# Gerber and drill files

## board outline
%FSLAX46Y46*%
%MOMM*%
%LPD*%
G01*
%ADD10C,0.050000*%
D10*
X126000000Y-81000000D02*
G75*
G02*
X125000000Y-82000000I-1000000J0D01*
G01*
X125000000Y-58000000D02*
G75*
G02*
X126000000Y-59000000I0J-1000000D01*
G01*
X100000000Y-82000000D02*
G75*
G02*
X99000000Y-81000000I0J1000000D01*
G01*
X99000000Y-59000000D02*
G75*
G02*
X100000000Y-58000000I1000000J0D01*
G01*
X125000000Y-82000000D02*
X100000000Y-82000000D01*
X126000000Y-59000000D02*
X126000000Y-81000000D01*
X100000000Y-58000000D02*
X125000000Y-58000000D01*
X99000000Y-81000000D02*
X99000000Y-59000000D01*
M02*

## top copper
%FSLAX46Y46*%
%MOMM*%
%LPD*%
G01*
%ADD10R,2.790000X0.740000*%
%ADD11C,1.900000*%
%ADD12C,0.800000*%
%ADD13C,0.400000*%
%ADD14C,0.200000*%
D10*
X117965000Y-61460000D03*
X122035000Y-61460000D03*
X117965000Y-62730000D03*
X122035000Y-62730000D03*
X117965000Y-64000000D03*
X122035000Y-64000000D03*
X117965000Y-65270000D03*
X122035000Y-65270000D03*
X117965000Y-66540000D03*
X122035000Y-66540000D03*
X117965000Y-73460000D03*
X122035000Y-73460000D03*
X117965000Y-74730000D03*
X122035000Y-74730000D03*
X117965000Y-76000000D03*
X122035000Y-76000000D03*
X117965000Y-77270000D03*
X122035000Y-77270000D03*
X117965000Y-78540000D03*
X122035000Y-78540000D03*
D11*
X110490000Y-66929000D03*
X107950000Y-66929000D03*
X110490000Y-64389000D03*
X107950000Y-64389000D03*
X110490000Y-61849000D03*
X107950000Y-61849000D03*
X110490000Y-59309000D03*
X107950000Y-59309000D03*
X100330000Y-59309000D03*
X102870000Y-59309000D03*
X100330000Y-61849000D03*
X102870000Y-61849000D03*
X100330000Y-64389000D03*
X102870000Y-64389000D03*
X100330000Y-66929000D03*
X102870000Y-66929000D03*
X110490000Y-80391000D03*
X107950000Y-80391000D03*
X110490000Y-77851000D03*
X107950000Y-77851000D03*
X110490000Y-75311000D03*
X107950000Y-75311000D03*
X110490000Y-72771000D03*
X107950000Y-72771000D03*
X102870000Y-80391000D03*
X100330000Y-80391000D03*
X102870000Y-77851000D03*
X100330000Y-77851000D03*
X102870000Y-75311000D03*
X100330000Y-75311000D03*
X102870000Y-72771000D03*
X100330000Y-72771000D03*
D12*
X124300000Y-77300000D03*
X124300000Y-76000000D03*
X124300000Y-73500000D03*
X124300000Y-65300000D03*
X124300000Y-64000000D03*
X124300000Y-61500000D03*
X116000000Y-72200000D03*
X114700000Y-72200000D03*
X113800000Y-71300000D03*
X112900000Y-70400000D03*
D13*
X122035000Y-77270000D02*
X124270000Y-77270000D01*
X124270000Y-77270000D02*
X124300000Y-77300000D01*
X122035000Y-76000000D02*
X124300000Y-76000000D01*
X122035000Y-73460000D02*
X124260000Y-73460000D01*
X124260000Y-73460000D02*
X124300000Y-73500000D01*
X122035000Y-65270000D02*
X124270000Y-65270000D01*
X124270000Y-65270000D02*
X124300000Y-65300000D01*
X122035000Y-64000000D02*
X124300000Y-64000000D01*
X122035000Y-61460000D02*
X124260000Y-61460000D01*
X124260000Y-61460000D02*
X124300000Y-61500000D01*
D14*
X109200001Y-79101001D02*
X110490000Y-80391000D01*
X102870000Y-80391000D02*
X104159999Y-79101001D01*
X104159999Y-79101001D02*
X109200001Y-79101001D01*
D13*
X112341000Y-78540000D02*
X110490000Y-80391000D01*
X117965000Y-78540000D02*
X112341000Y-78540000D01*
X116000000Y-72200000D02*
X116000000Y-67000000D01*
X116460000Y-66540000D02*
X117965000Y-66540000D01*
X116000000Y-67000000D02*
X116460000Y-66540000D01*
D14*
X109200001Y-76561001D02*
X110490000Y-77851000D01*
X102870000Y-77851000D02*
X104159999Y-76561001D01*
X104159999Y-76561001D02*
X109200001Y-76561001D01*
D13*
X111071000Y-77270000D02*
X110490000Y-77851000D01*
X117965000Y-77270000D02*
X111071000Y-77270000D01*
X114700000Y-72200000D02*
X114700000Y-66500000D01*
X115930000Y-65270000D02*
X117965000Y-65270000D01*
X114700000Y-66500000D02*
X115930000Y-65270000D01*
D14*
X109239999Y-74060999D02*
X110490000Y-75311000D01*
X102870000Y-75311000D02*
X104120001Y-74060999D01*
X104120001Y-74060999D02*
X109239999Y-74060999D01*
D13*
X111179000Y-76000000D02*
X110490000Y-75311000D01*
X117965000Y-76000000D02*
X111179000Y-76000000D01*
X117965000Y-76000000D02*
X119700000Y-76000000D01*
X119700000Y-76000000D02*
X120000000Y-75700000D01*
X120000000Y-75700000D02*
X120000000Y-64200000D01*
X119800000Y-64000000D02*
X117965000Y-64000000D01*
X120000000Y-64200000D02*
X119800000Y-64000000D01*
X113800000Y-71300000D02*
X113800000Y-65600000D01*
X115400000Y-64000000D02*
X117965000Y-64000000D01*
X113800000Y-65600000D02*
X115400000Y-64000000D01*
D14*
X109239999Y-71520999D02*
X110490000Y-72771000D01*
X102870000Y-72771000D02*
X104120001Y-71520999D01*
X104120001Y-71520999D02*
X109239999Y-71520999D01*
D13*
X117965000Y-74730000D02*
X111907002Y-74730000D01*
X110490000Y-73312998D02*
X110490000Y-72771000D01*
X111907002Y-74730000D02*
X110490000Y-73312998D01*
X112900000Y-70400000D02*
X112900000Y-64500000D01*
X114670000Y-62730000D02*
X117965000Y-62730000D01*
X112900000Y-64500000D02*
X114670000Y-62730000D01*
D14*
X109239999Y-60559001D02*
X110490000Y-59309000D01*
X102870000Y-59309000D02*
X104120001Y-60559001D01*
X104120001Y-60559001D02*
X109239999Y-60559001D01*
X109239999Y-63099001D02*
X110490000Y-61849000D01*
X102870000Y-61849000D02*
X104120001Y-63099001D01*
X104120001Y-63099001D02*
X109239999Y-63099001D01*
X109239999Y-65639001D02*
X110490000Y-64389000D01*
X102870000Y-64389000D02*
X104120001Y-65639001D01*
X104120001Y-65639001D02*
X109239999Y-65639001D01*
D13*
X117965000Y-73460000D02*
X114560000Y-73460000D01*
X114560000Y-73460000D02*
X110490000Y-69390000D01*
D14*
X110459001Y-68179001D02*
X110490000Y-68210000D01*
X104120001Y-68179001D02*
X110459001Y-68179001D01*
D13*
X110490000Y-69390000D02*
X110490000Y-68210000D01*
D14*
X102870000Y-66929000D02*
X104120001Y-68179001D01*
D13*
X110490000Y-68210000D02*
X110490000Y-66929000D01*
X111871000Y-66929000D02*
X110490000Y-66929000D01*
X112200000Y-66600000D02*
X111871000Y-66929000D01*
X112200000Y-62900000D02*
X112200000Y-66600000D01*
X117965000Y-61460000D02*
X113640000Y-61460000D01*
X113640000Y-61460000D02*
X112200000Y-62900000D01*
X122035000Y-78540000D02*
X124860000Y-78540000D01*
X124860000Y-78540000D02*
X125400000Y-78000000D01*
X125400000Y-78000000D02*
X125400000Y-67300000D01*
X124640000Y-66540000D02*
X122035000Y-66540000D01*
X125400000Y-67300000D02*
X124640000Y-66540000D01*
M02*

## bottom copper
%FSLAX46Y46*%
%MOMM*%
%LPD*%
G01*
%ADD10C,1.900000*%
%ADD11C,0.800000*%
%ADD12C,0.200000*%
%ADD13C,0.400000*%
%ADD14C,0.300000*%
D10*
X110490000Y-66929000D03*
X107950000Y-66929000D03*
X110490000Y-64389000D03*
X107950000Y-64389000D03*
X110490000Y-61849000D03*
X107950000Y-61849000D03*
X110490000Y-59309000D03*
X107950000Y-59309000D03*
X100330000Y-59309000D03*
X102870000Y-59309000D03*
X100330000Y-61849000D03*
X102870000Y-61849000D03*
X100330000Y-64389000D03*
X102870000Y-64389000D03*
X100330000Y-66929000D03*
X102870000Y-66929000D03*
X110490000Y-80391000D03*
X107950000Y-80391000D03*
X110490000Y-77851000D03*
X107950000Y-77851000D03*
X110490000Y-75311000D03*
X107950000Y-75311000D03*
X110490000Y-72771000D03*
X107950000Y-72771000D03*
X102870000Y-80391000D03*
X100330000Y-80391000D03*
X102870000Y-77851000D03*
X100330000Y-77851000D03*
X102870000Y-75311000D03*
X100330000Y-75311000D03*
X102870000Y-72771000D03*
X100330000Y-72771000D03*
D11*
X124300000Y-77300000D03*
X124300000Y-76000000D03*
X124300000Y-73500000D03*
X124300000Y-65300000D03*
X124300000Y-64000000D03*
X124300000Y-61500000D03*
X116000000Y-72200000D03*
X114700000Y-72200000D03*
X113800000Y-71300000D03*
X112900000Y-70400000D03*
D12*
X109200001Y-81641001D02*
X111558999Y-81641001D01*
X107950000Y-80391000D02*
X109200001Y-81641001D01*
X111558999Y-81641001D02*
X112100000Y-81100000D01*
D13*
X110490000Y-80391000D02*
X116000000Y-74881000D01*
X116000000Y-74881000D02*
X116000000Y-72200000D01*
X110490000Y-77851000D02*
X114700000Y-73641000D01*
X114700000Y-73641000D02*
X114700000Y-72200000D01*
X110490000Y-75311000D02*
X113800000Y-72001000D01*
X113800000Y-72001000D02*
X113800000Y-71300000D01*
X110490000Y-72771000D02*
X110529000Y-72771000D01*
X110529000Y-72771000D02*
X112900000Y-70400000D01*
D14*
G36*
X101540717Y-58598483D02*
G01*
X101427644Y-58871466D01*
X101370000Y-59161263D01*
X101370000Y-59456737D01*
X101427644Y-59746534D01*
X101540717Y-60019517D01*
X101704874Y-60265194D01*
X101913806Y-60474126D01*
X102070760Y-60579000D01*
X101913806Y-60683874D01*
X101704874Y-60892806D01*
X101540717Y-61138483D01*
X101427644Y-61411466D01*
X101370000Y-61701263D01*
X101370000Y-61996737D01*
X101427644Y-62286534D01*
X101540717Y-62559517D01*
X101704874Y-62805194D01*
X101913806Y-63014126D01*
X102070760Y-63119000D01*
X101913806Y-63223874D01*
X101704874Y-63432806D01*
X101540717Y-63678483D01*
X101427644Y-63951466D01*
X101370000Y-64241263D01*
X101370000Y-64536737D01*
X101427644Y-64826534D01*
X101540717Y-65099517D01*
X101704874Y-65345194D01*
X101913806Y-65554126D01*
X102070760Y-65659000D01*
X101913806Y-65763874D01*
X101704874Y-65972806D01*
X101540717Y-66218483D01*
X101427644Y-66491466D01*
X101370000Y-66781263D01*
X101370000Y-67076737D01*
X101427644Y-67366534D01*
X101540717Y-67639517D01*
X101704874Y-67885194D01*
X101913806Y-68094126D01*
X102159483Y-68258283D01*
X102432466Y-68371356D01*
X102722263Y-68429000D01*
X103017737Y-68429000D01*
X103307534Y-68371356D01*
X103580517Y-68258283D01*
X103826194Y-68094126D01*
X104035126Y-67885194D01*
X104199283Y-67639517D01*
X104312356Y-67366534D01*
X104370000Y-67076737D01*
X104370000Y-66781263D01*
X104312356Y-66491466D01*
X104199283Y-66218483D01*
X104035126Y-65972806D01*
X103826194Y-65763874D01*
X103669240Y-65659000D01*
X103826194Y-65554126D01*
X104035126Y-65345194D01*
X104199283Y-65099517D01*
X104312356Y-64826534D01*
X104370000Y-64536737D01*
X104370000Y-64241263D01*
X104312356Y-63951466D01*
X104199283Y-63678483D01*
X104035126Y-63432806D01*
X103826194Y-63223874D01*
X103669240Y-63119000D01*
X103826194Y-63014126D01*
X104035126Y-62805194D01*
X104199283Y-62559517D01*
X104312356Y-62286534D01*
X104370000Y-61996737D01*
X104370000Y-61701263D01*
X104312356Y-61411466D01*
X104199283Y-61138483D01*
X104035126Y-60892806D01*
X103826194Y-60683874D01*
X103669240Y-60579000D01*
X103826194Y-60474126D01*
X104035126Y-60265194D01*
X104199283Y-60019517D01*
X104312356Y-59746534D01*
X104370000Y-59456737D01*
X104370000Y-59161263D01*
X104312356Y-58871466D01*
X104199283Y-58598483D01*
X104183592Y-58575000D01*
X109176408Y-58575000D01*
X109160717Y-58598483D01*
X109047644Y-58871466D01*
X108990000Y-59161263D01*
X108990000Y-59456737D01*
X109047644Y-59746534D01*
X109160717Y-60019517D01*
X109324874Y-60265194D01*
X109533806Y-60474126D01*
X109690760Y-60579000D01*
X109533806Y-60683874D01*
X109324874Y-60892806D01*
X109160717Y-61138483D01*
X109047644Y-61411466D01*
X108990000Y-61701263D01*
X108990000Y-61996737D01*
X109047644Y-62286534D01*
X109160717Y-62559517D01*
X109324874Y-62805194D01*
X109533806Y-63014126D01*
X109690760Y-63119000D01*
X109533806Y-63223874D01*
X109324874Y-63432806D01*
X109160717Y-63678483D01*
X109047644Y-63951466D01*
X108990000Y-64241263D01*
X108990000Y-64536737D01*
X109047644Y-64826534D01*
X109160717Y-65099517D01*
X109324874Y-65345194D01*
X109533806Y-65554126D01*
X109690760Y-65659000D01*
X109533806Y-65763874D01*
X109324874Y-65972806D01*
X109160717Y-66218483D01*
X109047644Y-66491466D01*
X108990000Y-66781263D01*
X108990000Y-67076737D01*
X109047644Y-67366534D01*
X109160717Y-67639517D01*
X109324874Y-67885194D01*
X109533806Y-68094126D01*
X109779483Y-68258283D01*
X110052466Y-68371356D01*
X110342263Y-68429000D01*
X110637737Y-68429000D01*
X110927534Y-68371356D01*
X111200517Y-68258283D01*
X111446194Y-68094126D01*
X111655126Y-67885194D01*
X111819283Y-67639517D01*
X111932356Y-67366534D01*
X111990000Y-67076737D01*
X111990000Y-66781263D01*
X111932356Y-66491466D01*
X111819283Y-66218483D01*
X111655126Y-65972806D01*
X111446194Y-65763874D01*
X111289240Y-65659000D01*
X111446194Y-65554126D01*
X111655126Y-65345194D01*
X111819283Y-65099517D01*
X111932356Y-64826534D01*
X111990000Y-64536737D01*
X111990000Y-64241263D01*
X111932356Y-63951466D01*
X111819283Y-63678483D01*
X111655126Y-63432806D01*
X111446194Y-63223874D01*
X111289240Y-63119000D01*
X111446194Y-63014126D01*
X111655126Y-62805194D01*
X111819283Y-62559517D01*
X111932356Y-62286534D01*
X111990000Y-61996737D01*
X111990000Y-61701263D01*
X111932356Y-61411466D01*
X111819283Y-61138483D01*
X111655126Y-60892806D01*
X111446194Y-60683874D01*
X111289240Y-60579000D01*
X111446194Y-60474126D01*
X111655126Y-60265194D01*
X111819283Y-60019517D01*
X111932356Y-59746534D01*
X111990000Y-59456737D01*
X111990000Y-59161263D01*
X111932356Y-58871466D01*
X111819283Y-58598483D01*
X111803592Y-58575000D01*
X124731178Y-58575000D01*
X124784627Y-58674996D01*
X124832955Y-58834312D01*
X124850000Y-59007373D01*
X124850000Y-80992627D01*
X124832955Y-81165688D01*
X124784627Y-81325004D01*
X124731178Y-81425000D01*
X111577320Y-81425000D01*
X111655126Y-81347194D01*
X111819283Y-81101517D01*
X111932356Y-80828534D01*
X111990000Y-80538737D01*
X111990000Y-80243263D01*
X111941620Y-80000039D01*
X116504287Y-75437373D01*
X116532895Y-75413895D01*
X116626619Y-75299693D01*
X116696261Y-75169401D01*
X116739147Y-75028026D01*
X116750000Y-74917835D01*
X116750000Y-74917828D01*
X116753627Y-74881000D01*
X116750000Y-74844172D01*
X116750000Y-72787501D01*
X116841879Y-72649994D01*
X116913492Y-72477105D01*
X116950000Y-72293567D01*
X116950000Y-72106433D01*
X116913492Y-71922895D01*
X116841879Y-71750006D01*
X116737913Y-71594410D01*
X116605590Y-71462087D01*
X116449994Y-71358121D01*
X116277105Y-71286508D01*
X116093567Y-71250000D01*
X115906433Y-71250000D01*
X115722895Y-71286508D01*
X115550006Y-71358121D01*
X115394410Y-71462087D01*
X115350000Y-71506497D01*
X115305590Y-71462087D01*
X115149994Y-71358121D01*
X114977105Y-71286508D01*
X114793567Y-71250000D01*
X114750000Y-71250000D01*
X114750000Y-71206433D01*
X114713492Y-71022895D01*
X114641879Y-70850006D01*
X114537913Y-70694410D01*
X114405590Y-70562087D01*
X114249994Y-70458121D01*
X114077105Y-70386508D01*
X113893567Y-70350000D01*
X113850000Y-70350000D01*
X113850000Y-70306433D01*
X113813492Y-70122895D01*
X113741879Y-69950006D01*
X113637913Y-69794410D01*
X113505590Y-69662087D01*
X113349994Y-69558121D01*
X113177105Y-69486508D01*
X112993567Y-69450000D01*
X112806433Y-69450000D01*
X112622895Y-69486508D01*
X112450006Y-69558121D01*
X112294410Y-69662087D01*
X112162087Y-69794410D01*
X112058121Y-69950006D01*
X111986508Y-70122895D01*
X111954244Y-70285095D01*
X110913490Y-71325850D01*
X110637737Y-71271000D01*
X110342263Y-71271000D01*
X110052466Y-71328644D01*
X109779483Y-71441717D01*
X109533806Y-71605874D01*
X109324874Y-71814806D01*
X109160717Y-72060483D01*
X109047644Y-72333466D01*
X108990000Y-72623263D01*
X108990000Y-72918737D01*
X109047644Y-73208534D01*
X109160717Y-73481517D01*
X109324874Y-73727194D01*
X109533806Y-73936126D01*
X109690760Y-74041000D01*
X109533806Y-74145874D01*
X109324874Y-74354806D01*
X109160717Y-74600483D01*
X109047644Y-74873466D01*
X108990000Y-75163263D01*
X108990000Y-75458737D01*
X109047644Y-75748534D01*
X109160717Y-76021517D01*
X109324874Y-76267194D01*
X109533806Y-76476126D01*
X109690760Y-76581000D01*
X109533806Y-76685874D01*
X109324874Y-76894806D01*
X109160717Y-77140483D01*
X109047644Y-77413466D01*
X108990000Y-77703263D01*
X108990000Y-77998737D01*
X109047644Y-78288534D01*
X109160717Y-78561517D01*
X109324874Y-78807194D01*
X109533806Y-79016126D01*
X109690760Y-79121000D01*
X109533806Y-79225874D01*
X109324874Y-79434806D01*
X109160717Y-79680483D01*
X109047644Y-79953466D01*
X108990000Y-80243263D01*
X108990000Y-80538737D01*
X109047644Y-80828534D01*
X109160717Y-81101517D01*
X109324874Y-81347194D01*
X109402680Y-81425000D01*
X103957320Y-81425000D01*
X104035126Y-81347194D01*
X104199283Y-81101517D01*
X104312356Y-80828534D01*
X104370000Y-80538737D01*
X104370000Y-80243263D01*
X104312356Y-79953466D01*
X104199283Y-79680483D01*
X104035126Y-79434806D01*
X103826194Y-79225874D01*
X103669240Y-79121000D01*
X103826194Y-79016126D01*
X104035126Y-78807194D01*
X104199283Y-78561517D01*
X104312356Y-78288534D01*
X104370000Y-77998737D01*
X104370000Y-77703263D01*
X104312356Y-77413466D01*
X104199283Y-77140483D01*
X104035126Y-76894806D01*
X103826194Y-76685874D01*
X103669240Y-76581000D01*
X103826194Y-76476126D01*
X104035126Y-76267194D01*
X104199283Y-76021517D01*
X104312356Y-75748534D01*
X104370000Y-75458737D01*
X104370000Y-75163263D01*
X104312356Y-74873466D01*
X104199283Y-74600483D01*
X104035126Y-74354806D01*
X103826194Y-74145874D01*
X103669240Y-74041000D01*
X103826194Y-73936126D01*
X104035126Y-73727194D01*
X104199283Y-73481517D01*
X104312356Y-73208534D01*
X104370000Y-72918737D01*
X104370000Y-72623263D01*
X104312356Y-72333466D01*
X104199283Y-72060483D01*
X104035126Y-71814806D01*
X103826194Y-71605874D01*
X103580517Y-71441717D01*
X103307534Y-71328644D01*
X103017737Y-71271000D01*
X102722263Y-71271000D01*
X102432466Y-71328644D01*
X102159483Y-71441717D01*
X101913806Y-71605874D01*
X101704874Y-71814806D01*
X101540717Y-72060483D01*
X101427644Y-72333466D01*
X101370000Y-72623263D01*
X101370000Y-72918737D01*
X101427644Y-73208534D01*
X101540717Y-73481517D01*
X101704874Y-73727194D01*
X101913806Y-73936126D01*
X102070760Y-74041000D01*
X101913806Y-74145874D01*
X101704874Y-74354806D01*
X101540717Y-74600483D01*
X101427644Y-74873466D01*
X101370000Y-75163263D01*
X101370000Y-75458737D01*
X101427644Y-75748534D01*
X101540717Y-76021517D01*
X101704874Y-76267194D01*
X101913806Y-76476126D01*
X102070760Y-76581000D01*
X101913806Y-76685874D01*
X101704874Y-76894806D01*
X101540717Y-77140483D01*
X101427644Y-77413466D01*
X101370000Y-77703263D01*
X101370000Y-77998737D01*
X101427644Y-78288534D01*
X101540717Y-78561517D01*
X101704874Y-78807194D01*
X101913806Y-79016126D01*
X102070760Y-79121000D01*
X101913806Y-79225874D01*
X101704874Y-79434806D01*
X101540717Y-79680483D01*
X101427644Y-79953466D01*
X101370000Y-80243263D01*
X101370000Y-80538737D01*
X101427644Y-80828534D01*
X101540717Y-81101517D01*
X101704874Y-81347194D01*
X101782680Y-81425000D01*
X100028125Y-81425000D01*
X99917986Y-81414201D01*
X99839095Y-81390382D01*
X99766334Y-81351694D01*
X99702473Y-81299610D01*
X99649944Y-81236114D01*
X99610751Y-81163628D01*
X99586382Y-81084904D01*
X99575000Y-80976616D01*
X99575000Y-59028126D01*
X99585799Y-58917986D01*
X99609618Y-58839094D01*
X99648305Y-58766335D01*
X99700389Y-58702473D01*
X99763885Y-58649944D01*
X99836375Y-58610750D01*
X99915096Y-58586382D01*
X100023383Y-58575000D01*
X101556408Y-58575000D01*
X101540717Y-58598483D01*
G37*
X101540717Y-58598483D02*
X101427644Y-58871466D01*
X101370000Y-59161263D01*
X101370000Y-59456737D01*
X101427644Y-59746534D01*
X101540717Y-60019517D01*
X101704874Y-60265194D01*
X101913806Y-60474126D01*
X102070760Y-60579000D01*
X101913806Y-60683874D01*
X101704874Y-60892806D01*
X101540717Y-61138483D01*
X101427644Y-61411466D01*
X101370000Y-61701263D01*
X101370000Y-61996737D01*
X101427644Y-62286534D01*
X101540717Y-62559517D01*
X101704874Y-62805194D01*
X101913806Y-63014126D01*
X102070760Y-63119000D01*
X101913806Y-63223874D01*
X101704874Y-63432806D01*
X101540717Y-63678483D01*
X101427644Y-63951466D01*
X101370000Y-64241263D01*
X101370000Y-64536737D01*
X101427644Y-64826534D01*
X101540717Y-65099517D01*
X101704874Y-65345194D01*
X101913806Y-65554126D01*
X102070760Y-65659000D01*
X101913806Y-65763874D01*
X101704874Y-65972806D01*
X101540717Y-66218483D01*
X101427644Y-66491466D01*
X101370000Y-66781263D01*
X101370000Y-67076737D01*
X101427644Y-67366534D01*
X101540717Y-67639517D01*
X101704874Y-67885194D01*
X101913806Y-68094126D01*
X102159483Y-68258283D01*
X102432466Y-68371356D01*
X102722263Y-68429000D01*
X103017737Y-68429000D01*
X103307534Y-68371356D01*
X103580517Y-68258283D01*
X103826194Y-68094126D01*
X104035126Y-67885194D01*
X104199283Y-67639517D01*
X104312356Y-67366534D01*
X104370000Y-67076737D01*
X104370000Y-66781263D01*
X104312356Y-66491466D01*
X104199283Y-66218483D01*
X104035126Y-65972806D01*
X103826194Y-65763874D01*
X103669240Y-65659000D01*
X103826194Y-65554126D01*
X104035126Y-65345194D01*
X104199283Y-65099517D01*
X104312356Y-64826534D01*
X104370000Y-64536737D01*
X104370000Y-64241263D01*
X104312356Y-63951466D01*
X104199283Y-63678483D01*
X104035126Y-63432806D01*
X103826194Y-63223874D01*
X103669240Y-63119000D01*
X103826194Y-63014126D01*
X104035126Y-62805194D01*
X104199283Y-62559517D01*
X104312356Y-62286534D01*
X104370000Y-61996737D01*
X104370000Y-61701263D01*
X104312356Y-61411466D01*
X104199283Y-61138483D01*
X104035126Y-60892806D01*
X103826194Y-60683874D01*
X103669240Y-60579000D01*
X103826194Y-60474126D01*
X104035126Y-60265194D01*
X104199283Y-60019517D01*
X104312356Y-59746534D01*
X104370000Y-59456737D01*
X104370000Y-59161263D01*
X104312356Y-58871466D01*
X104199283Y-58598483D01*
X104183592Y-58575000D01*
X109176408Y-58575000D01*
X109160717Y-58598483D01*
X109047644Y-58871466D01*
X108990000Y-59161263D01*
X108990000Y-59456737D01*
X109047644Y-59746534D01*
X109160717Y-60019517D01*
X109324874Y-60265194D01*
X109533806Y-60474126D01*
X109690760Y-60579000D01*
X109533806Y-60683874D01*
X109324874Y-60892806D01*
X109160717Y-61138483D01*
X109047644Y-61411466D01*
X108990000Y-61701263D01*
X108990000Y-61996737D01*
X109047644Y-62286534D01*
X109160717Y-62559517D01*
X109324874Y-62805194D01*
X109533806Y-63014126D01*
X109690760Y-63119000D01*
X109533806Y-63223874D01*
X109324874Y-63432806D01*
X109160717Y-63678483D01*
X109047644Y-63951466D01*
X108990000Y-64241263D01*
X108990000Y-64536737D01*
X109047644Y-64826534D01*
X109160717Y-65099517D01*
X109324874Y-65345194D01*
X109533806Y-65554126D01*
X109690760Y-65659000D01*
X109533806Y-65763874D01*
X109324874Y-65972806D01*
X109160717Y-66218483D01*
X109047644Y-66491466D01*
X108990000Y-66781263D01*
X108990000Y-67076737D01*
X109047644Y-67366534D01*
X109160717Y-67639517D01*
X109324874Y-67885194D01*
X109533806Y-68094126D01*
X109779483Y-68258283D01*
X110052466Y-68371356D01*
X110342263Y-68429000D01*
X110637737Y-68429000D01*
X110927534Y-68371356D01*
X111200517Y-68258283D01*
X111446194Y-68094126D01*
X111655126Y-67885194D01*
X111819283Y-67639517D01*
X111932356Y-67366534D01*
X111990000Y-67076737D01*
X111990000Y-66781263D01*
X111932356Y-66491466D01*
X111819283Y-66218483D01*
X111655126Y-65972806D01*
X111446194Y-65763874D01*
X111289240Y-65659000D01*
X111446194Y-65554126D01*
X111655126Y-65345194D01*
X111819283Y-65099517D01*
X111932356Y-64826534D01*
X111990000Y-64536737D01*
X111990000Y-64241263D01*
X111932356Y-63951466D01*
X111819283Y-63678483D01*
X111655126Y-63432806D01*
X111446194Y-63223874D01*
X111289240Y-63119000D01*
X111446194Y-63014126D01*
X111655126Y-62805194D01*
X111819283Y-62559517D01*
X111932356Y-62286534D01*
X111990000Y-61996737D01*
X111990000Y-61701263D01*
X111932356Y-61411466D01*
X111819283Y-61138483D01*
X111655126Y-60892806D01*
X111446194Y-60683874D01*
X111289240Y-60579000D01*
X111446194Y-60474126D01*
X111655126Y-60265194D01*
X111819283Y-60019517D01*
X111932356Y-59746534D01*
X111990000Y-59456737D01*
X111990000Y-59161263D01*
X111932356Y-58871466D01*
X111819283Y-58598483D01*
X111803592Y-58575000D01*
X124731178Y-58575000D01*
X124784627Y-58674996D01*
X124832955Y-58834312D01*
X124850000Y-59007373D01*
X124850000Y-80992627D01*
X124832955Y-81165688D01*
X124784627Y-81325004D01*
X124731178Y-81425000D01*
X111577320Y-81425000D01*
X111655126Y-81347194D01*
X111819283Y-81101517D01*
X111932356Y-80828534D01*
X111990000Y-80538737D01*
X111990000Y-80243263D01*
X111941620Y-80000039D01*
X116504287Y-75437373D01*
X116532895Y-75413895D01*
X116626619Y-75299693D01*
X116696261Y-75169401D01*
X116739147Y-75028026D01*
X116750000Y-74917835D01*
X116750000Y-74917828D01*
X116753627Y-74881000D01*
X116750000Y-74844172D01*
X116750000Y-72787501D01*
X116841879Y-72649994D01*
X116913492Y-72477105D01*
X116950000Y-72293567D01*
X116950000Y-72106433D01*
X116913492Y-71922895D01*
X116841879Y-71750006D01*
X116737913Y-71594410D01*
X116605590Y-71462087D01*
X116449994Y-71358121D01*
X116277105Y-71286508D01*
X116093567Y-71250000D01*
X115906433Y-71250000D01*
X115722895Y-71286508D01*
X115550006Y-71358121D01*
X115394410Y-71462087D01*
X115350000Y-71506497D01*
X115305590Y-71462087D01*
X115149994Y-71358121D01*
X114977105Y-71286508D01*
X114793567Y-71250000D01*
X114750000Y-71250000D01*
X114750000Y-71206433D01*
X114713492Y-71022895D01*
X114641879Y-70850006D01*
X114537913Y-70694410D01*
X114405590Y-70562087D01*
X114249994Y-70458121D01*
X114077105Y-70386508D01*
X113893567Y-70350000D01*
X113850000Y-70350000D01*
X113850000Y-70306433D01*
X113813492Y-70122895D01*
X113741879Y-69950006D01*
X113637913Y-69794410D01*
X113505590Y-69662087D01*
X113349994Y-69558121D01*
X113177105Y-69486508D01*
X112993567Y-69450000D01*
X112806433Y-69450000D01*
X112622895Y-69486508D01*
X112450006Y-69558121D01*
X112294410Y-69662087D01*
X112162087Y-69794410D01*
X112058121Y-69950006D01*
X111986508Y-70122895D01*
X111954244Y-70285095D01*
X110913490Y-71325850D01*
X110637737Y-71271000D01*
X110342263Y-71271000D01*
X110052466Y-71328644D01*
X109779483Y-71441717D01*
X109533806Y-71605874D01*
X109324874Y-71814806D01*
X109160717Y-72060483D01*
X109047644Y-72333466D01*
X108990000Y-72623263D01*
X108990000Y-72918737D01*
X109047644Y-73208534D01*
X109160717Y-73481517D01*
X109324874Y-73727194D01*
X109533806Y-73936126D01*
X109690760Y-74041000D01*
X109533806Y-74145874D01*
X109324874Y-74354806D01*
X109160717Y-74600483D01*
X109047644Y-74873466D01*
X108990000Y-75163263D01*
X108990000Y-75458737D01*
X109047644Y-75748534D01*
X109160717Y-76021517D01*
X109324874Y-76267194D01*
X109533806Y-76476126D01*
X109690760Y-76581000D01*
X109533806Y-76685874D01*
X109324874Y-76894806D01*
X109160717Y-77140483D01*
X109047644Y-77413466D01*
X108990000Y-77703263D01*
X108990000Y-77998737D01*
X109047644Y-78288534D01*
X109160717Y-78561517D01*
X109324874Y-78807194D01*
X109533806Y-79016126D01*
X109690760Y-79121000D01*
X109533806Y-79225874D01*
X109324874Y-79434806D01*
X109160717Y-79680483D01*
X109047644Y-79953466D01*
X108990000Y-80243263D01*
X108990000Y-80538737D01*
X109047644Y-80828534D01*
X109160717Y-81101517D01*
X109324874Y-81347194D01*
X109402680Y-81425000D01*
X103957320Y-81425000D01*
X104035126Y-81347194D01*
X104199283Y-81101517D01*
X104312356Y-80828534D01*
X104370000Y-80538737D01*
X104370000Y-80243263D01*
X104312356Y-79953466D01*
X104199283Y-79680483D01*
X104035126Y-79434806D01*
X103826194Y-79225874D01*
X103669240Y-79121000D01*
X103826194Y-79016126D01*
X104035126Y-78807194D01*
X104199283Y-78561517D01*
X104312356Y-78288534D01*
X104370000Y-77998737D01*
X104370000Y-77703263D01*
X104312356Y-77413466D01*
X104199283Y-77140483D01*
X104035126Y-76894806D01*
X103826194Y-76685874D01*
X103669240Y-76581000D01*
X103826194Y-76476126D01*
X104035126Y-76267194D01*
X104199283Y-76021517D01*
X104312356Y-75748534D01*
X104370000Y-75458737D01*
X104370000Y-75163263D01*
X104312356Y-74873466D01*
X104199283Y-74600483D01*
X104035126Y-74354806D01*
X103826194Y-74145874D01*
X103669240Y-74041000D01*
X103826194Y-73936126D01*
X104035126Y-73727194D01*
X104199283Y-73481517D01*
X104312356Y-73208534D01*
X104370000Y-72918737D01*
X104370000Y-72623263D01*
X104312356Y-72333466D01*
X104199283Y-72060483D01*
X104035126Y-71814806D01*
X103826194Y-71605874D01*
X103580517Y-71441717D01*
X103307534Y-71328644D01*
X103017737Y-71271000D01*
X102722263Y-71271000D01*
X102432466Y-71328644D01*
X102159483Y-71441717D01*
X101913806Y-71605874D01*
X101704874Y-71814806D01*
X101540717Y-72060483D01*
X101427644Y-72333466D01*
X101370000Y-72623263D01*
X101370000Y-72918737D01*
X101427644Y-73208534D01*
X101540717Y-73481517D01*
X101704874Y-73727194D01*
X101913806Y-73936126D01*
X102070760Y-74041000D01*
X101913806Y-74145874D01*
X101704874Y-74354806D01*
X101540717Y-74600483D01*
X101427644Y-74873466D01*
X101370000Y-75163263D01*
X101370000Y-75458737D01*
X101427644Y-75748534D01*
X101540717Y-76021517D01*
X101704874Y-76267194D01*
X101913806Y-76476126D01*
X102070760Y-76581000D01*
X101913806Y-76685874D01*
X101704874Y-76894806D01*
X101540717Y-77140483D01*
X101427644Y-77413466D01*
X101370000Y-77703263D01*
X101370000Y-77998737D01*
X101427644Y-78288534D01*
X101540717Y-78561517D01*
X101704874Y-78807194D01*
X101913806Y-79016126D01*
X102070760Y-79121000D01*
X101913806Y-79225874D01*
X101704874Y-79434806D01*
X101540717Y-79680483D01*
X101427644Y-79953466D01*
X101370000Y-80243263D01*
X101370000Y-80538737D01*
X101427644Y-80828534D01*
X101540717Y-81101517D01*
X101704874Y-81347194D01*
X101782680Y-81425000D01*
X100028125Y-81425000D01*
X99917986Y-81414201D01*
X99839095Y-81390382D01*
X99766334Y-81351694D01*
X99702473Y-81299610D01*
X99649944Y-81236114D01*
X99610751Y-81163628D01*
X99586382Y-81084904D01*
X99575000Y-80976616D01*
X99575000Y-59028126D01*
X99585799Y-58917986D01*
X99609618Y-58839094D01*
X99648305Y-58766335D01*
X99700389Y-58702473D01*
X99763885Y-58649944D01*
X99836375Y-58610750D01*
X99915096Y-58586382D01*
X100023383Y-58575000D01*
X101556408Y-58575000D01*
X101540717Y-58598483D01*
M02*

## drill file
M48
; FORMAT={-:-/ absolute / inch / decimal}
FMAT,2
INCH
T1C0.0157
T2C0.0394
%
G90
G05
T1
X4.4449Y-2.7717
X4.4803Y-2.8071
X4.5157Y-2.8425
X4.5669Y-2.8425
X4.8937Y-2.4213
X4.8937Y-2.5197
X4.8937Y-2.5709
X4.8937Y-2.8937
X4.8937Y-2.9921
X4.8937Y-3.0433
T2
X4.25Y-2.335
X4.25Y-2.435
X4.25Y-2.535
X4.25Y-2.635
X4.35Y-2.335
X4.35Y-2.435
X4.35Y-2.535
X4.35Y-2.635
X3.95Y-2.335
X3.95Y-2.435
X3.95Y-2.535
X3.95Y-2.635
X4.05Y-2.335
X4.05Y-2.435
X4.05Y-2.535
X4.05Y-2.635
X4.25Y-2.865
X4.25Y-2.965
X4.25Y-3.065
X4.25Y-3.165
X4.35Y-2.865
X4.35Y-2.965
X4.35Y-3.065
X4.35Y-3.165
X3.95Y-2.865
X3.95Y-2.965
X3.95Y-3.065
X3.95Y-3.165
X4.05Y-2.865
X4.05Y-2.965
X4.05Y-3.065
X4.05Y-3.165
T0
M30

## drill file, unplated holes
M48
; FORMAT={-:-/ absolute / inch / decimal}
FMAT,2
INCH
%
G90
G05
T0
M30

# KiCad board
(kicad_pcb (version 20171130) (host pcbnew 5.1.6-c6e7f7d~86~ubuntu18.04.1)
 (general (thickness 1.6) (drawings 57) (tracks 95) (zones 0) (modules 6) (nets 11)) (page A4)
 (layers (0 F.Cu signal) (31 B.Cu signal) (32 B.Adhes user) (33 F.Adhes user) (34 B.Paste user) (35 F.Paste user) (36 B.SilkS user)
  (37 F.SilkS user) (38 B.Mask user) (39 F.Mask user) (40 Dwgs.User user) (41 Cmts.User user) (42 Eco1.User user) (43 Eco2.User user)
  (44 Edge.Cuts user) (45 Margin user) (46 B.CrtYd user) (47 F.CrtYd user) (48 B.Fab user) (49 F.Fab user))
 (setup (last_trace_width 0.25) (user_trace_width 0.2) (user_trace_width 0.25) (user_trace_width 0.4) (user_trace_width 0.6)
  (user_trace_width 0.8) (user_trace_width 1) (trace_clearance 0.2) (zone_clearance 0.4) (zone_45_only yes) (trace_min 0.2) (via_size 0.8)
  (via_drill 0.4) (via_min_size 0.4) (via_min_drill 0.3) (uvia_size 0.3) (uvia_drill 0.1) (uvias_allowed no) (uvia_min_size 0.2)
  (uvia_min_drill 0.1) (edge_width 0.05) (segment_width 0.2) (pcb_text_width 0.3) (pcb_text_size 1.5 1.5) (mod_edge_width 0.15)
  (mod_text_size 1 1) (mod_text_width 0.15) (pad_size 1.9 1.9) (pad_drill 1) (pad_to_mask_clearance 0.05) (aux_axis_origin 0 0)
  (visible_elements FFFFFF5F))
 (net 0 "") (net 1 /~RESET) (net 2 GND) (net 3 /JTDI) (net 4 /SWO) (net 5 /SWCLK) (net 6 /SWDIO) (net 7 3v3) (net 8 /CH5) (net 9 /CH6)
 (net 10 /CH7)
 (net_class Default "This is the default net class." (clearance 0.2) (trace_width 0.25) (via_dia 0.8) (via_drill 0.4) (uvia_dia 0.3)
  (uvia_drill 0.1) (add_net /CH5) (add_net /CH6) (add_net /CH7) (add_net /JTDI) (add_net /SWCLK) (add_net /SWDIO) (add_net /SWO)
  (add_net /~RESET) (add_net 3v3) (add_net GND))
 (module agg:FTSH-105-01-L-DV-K (layer F.Cu) (at 120 64 90)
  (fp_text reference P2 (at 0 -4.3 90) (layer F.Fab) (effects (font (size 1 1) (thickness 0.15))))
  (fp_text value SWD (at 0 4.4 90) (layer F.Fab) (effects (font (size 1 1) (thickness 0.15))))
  (pad 10 smd rect (at 2.54 -2.035 90) (size 0.74 2.79) (layers F.Cu F.Paste F.Mask) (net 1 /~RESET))
  (pad 9 smd rect (at 2.54 2.035 90) (size 0.74 2.79) (layers F.Cu F.Paste F.Mask) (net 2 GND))
  (pad 8 smd rect (at 1.27 -2.035 90) (size 0.74 2.79) (layers F.Cu F.Paste F.Mask) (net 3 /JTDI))
  (pad 7 smd rect (at 1.27 2.035 90) (size 0.74 2.79) (layers F.Cu F.Paste F.Mask))
  (pad 6 smd rect (at 0 -2.035 90) (size 0.74 2.79) (layers F.Cu F.Paste F.Mask) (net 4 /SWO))
  (pad 5 smd rect (at 0 2.035 90) (size 0.74 2.79) (layers F.Cu F.Paste F.Mask) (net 2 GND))
  (pad 4 smd rect (at -1.27 -2.035 90) (size 0.74 2.79) (layers F.Cu F.Paste F.Mask) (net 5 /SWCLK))
  (pad 3 smd rect (at -1.27 2.035 90) (size 0.74 2.79) (layers F.Cu F.Paste F.Mask) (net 2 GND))
  (pad 2 smd rect (at -2.54 -2.035 90) (size 0.74 2.79) (layers F.Cu F.Paste F.Mask) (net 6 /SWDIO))
  (pad 1 smd rect (at -2.54 2.035 90) (size 0.74 2.79) (layers F.Cu F.Paste F.Mask) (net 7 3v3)))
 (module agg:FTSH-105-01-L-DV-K (layer F.Cu) (at 120 76 90)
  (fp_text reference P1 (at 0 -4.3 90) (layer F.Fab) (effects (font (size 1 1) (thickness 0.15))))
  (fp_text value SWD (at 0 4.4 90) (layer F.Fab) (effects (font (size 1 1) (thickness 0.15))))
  (pad 10 smd rect (at 2.54 -2.035 90) (size 0.74 2.79) (layers F.Cu F.Paste F.Mask) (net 1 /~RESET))
  (pad 9 smd rect (at 2.54 2.035 90) (size 0.74 2.79) (layers F.Cu F.Paste F.Mask) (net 2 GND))
  (pad 8 smd rect (at 1.27 -2.035 90) (size 0.74 2.79) (layers F.Cu F.Paste F.Mask) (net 3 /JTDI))
  (pad 7 smd rect (at 1.27 2.035 90) (size 0.74 2.79) (layers F.Cu F.Paste F.Mask))
  (pad 6 smd rect (at 0 -2.035 90) (size 0.74 2.79) (layers F.Cu F.Paste F.Mask) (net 4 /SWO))
  (pad 5 smd rect (at 0 2.035 90) (size 0.74 2.79) (layers F.Cu F.Paste F.Mask) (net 2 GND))
  (pad 4 smd rect (at -1.27 -2.035 90) (size 0.74 2.79) (layers F.Cu F.Paste F.Mask) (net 5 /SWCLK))
  (pad 3 smd rect (at -1.27 2.035 90) (size 0.74 2.79) (layers F.Cu F.Paste F.Mask) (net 2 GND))
  (pad 2 smd rect (at -2.54 -2.035 90) (size 0.74 2.79) (layers F.Cu F.Paste F.Mask) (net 6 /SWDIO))
  (pad 1 smd rect (at -2.54 2.035 90) (size 0.74 2.79) (layers F.Cu F.Paste F.Mask) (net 7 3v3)))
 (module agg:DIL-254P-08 (layer F.Cu) (at 109.22 63.119 270)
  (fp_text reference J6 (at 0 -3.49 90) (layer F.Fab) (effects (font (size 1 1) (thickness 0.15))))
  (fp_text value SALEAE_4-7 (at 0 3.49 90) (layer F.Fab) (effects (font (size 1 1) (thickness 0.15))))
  (pad 8 thru_hole circle (at 3.81 -1.27 270) (size 1.9 1.9) (drill 1) (layers *.Cu *.Mask F.SilkS) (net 1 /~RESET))
  (pad 7 thru_hole circle (at 3.81 1.27 270) (size 1.9 1.9) (drill 1) (layers *.Cu *.Mask F.SilkS) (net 2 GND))
  (pad 6 thru_hole circle (at 1.27 -1.27 270) (size 1.9 1.9) (drill 1) (layers *.Cu *.Mask F.SilkS) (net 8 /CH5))
  (pad 5 thru_hole circle (at 1.27 1.27 270) (size 1.9 1.9) (drill 1) (layers *.Cu *.Mask F.SilkS) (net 2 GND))
  (pad 4 thru_hole circle (at -1.27 -1.27 270) (size 1.9 1.9) (drill 1) (layers *.Cu *.Mask F.SilkS) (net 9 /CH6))
  (pad 3 thru_hole circle (at -1.27 1.27 270) (size 1.9 1.9) (drill 1) (layers *.Cu *.Mask F.SilkS) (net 2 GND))
  (pad 2 thru_hole circle (at -3.81 -1.27 270) (size 1.9 1.9) (drill 1) (layers *.Cu *.Mask F.SilkS) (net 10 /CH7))
  (pad 1 thru_hole circle (at -3.81 1.27 270) (size 1.9 1.9) (drill 1) (layers *.Cu *.Mask F.SilkS) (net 2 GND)))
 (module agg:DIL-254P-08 (layer F.Cu) (at 101.6 63.119 270)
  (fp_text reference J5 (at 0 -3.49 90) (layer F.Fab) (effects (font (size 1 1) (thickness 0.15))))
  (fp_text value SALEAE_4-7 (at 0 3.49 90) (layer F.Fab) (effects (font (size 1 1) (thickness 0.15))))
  (pad 1 thru_hole circle (at -3.81 1.27 270) (size 1.9 1.9) (drill 1) (layers *.Cu *.Mask F.SilkS) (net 2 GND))
  (pad 2 thru_hole circle (at -3.81 -1.27 270) (size 1.9 1.9) (drill 1) (layers *.Cu *.Mask F.SilkS) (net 10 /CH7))
  (pad 3 thru_hole circle (at -1.27 1.27 270) (size 1.9 1.9) (drill 1) (layers *.Cu *.Mask F.SilkS) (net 2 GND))
  (pad 4 thru_hole circle (at -1.27 -1.27 270) (size 1.9 1.9) (drill 1) (layers *.Cu *.Mask F.SilkS) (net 9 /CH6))
  (pad 5 thru_hole circle (at 1.27 1.27 270) (size 1.9 1.9) (drill 1) (layers *.Cu *.Mask F.SilkS) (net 2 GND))
  (pad 6 thru_hole circle (at 1.27 -1.27 270) (size 1.9 1.9) (drill 1) (layers *.Cu *.Mask F.SilkS) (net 8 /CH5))
  (pad 7 thru_hole circle (at 3.81 1.27 270) (size 1.9 1.9) (drill 1) (layers *.Cu *.Mask F.SilkS) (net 2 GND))
  (pad 8 thru_hole circle (at 3.81 -1.27 270) (size 1.9 1.9) (drill 1) (layers *.Cu *.Mask F.SilkS) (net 1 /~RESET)))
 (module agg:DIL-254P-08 (layer F.Cu) (at 109.22 76.581 270)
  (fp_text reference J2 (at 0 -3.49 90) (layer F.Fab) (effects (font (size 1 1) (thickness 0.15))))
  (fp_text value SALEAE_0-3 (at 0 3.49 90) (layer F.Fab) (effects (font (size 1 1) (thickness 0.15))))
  (pad 8 thru_hole circle (at 3.81 -1.27 270) (size 1.9 1.9) (drill 1) (layers *.Cu *.Mask F.SilkS) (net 6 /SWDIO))
  (pad 7 thru_hole circle (at 3.81 1.27 270) (size 1.9 1.9) (drill 1) (layers *.Cu *.Mask F.SilkS) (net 2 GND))
  (pad 6 thru_hole circle (at 1.27 -1.27 270) (size 1.9 1.9) (drill 1) (layers *.Cu *.Mask F.SilkS) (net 5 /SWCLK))
  (pad 5 thru_hole circle (at 1.27 1.27 270) (size 1.9 1.9) (drill 1) (layers *.Cu *.Mask F.SilkS) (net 2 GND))
  (pad 4 thru_hole circle (at -1.27 -1.27 270) (size 1.9 1.9) (drill 1) (layers *.Cu *.Mask F.SilkS) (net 4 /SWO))
  (pad 3 thru_hole circle (at -1.27 1.27 270) (size 1.9 1.9) (drill 1) (layers *.Cu *.Mask F.SilkS) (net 2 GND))
  (pad 2 thru_hole circle (at -3.81 -1.27 270) (size 1.9 1.9) (drill 1) (layers *.Cu *.Mask F.SilkS) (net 3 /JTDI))
  (pad 1 thru_hole circle (at -3.81 1.27 270) (size 1.9 1.9) (drill 1) (layers *.Cu *.Mask F.SilkS) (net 2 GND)))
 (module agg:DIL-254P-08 (layer F.Cu) (at 101.6 76.581 270)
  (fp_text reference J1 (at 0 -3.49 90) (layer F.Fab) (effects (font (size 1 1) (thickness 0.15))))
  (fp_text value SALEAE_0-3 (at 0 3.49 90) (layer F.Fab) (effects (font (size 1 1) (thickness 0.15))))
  (pad 8 thru_hole circle (at 3.81 -1.27 270) (size 1.9 1.9) (drill 1) (layers *.Cu *.Mask F.SilkS) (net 6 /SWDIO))
  (pad 7 thru_hole circle (at 3.81 1.27 270) (size 1.9 1.9) (drill 1) (layers *.Cu *.Mask F.SilkS) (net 2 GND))
  (pad 6 thru_hole circle (at 1.27 -1.27 270) (size 1.9 1.9) (drill 1) (layers *.Cu *.Mask F.SilkS) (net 5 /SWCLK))
  (pad 5 thru_hole circle (at 1.27 1.27 270) (size 1.9 1.9) (drill 1) (layers *.Cu *.Mask F.SilkS) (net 2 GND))
  (pad 4 thru_hole circle (at -1.27 -1.27 270) (size 1.9 1.9) (drill 1) (layers *.Cu *.Mask F.SilkS) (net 4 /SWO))
  (pad 3 thru_hole circle (at -1.27 1.27 270) (size 1.9 1.9) (drill 1) (layers *.Cu *.Mask F.SilkS) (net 2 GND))
  (pad 2 thru_hole circle (at -3.81 -1.27 270) (size 1.9 1.9) (drill 1) (layers *.Cu *.Mask F.SilkS) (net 3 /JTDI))
  (pad 1 thru_hole circle (at -3.81 1.27 270) (size 1.9 1.9) (drill 1) (layers *.Cu *.Mask F.SilkS) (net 2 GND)))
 (gr_arc (start 125 81) (end 125 82) (angle -90) (layer Edge.Cuts) (width 0.05))
 (gr_arc (start 125 59) (end 126 59) (angle -90) (layer Edge.Cuts) (width 0.05))
 (gr_arc (start 100 81) (end 99 81) (angle -90) (layer Edge.Cuts) (width 0.05))
 (gr_arc (start 100 59) (end 100 58) (angle -90) (layer Edge.Cuts) (width 0.05))
 (gr_line (start 125 82) (end 100 82) (layer Edge.Cuts) (width 0.05))
 (gr_line (start 126 59) (end 126 81) (layer Edge.Cuts) (width 0.05))
 (gr_line (start 100 58) (end 125 58) (layer Edge.Cuts) (width 0.05))
 (gr_line (start 99 81) (end 99 59) (layer Edge.Cuts) (width 0.05))
 (via (at 124.3 77.3) (size 0.8) (drill 0.4) (layers F.Cu B.Cu) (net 2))
 (segment (start 122.035 77.27) (end 124.27 77.27) (width 0.4) (layer F.Cu) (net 2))
 (segment (start 124.27 77.27) (end 124.3 77.3) (width 0.4) (layer F.Cu) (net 2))
 (via (at 124.3 76) (size 0.8) (drill 0.4) (layers F.Cu B.Cu) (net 2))
 (segment (start 122.035 76) (end 124.3 76) (width 0.4) (layer F.Cu) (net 2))
 (via (at 124.3 73.5) (size 0.8) (drill 0.4) (layers F.Cu B.Cu) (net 2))
 (segment (start 122.035 73.46) (end 124.26 73.46) (width 0.4) (layer F.Cu) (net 2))
 (segment (start 124.26 73.46) (end 124.3 73.5) (width 0.4) (layer F.Cu) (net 2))
 (segment (start 122.035 65.27) (end 124.27 65.27) (width 0.4) (layer F.Cu) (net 2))
 (via (at 124.3 65.3) (size 0.8) (drill 0.4) (layers F.Cu B.Cu) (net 2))
 (segment (start 124.27 65.27) (end 124.3 65.3) (width 0.4) (layer F.Cu) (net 2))
 (via (at 124.3 64) (size 0.8) (drill 0.4) (layers F.Cu B.Cu) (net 2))
 (segment (start 122.035 64) (end 124.3 64) (width 0.4) (layer F.Cu) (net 2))
 (via (at 124.3 61.5) (size 0.8) (drill 0.4) (layers F.Cu B.Cu) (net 2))
 (segment (start 122.035 61.46) (end 124.26 61.46) (width 0.4) (layer F.Cu) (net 2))
 (segment (start 124.26 61.46) (end 124.3 61.5) (width 0.4) (layer F.Cu) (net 2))
 (segment (start 109.200001 81.641001) (end 111.558999 81.641001) (width 0.2) (layer B.Cu) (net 2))
 (segment (start 107.95 80.391) (end 109.200001 81.641001) (width 0.2) (layer B.Cu) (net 2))
 (segment (start 111.558999 81.641001) (end 112.1 81.1) (width 0.2) (layer B.Cu) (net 2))
 (segment (start 109.200001 79.101001) (end 110.49 80.391) (width 0.2) (layer F.Cu) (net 6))
 (segment (start 102.87 80.391) (end 104.159999 79.101001) (width 0.2) (layer F.Cu) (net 6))
 (segment (start 104.159999 79.101001) (end 109.200001 79.101001) (width 0.2) (layer F.Cu) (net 6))
 (segment (start 112.341 78.54) (end 110.49 80.391) (width 0.4) (layer F.Cu) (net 6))
 (segment (start 117.965 78.54) (end 112.341 78.54) (width 0.4) (layer F.Cu) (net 6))
 (via (at 116 72.2) (size 0.8) (drill 0.4) (layers F.Cu B.Cu) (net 6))
 (segment (start 110.49 80.391) (end 116 74.881) (width 0.4) (layer B.Cu) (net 6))
 (segment (start 116 74.881) (end 116 72.2) (width 0.4) (layer B.Cu) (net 6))
 (segment (start 116 72.2) (end 116 67) (width 0.4) (layer F.Cu) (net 6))
 (segment (start 116.46 66.54) (end 117.965 66.54) (width 0.4) (layer F.Cu) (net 6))
 (segment (start 116 67) (end 116.46 66.54) (width 0.4) (layer F.Cu) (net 6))
 (segment (start 109.200001 76.561001) (end 110.49 77.851) (width 0.2) (layer F.Cu) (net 5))
 (segment (start 102.87 77.851) (end 104.159999 76.561001) (width 0.2) (layer F.Cu) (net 5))
 (segment (start 104.159999 76.561001) (end 109.200001 76.561001) (width 0.2) (layer F.Cu) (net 5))
 (segment (start 111.071 77.27) (end 110.49 77.851) (width 0.4) (layer F.Cu) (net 5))
 (segment (start 117.965 77.27) (end 111.071 77.27) (width 0.4) (layer F.Cu) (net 5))
 (via (at 114.7 72.2) (size 0.8) (drill 0.4) (layers F.Cu B.Cu) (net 5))
 (segment (start 110.49 77.851) (end 114.7 73.641) (width 0.4) (layer B.Cu) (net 5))
 (segment (start 114.7 73.641) (end 114.7 72.2) (width 0.4) (layer B.Cu) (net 5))
 (segment (start 114.7 72.2) (end 114.7 66.5) (width 0.4) (layer F.Cu) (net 5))
 (segment (start 115.93 65.27) (end 117.965 65.27) (width 0.4) (layer F.Cu) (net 5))
 (segment (start 114.7 66.5) (end 115.93 65.27) (width 0.4) (layer F.Cu) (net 5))
 (segment (start 109.239999 74.060999) (end 110.49 75.311) (width 0.2) (layer F.Cu) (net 4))
 (segment (start 102.87 75.311) (end 104.120001 74.060999) (width 0.2) (layer F.Cu) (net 4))
 (segment (start 104.120001 74.060999) (end 109.239999 74.060999) (width 0.2) (layer F.Cu) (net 4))
 (segment (start 111.179 76) (end 110.49 75.311) (width 0.4) (layer F.Cu) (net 4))
 (segment (start 117.965 76) (end 111.179 76) (width 0.4) (layer F.Cu) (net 4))
 (segment (start 117.965 76) (end 119.7 76) (width 0.4) (layer F.Cu) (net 4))
 (segment (start 119.7 76) (end 120 75.7) (width 0.4) (layer F.Cu) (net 4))
 (segment (start 120 75.7) (end 120 64.2) (width 0.4) (layer F.Cu) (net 4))
 (segment (start 119.8 64) (end 117.965 64) (width 0.4) (layer F.Cu) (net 4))
 (segment (start 120 64.2) (end 119.8 64) (width 0.4) (layer F.Cu) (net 4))
 (via (at 113.8 71.3) (size 0.8) (drill 0.4) (layers F.Cu B.Cu) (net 4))
 (segment (start 110.49 75.311) (end 113.8 72.001) (width 0.4) (layer B.Cu) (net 4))
 (segment (start 113.8 72.001) (end 113.8 71.3) (width 0.4) (layer B.Cu) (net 4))
 (segment (start 113.8 71.3) (end 113.8 65.6) (width 0.4) (layer F.Cu) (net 4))
 (segment (start 115.4 64) (end 117.965 64) (width 0.4) (layer F.Cu) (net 4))
 (segment (start 113.8 65.6) (end 115.4 64) (width 0.4) (layer F.Cu) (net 4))
 (segment (start 109.239999 71.520999) (end 110.49 72.771) (width 0.2) (layer F.Cu) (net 3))
 (segment (start 102.87 72.771) (end 104.120001 71.520999) (width 0.2) (layer F.Cu) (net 3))
 (segment (start 104.120001 71.520999) (end 109.239999 71.520999) (width 0.2) (layer F.Cu) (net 3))
 (segment (start 117.965 74.73) (end 111.907002 74.73) (width 0.4) (layer F.Cu) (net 3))
 (segment (start 110.49 73.312998) (end 110.49 72.771) (width 0.4) (layer F.Cu) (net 3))
 (segment (start 111.907002 74.73) (end 110.49 73.312998) (width 0.4) (layer F.Cu) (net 3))
 (segment (start 110.49 72.771) (end 110.529 72.771) (width 0.4) (layer B.Cu) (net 3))
 (via (at 112.9 70.4) (size 0.8) (drill 0.4) (layers F.Cu B.Cu) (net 3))
 (segment (start 110.529 72.771) (end 112.9 70.4) (width 0.4) (layer B.Cu) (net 3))
 (segment (start 112.9 70.4) (end 112.9 64.5) (width 0.4) (layer F.Cu) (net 3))
 (segment (start 114.67 62.73) (end 117.965 62.73) (width 0.4) (layer F.Cu) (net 3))
 (segment (start 112.9 64.5) (end 114.67 62.73) (width 0.4) (layer F.Cu) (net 3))
 (segment (start 109.239999 60.559001) (end 110.49 59.309) (width 0.2) (layer F.Cu) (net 10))
 (segment (start 102.87 59.309) (end 104.120001 60.559001) (width 0.2) (layer F.Cu) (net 10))
 (segment (start 104.120001 60.559001) (end 109.239999 60.559001) (width 0.2) (layer F.Cu) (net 10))
 (segment (start 109.239999 63.099001) (end 110.49 61.849) (width 0.2) (layer F.Cu) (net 9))
 (segment (start 102.87 61.849) (end 104.120001 63.099001) (width 0.2) (layer F.Cu) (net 9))
 (segment (start 104.120001 63.099001) (end 109.239999 63.099001) (width 0.2) (layer F.Cu) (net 9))
 (segment (start 109.239999 65.639001) (end 110.49 64.389) (width 0.2) (layer F.Cu) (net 8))
 (segment (start 102.87 64.389) (end 104.120001 65.639001) (width 0.2) (layer F.Cu) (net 8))
 (segment (start 104.120001 65.639001) (end 109.239999 65.639001) (width 0.2) (layer F.Cu) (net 8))
 (segment (start 117.965 73.46) (end 114.56 73.46) (width 0.4) (layer F.Cu) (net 1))
 (segment (start 114.56 73.46) (end 110.49 69.39) (width 0.4) (layer F.Cu) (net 1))
 (segment (start 110.459001 68.179001) (end 110.49 68.21) (width 0.2) (layer F.Cu) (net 1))
 (segment (start 104.120001 68.179001) (end 110.459001 68.179001) (width 0.2) (layer F.Cu) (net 1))
 (segment (start 110.49 69.39) (end 110.49 68.21) (width 0.4) (layer F.Cu) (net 1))
 (segment (start 102.87 66.929) (end 104.120001 68.179001) (width 0.2) (layer F.Cu) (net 1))
 (segment (start 110.49 68.21) (end 110.49 66.929) (width 0.4) (layer F.Cu) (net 1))
 (segment (start 111.871 66.929) (end 110.49 66.929) (width 0.4) (layer F.Cu) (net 1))
 (segment (start 112.2 66.6) (end 111.871 66.929) (width 0.4) (layer F.Cu) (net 1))
 (segment (start 112.2 62.9) (end 112.2 66.6) (width 0.4) (layer F.Cu) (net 1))
 (segment (start 117.965 61.46) (end 113.64 61.46) (width 0.4) (layer F.Cu) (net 1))
 (segment (start 113.64 61.46) (end 112.2 62.9) (width 0.4) (layer F.Cu) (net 1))
 (segment (start 122.035 78.54) (end 124.86 78.54) (width 0.4) (layer F.Cu) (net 7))
 (segment (start 124.86 78.54) (end 125.4 78) (width 0.4) (layer F.Cu) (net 7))
 (segment (start 125.4 78) (end 125.4 67.3) (width 0.4) (layer F.Cu) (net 7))
 (segment (start 124.64 66.54) (end 122.035 66.54) (width 0.4) (layer F.Cu) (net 7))
 (segment (start 125.4 67.3) (end 124.64 66.54) (width 0.4) (layer F.Cu) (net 7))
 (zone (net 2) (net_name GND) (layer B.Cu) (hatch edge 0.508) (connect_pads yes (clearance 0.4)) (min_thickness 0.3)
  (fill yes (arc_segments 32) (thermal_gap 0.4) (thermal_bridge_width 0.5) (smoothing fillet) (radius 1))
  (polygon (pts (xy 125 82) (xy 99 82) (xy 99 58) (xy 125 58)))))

